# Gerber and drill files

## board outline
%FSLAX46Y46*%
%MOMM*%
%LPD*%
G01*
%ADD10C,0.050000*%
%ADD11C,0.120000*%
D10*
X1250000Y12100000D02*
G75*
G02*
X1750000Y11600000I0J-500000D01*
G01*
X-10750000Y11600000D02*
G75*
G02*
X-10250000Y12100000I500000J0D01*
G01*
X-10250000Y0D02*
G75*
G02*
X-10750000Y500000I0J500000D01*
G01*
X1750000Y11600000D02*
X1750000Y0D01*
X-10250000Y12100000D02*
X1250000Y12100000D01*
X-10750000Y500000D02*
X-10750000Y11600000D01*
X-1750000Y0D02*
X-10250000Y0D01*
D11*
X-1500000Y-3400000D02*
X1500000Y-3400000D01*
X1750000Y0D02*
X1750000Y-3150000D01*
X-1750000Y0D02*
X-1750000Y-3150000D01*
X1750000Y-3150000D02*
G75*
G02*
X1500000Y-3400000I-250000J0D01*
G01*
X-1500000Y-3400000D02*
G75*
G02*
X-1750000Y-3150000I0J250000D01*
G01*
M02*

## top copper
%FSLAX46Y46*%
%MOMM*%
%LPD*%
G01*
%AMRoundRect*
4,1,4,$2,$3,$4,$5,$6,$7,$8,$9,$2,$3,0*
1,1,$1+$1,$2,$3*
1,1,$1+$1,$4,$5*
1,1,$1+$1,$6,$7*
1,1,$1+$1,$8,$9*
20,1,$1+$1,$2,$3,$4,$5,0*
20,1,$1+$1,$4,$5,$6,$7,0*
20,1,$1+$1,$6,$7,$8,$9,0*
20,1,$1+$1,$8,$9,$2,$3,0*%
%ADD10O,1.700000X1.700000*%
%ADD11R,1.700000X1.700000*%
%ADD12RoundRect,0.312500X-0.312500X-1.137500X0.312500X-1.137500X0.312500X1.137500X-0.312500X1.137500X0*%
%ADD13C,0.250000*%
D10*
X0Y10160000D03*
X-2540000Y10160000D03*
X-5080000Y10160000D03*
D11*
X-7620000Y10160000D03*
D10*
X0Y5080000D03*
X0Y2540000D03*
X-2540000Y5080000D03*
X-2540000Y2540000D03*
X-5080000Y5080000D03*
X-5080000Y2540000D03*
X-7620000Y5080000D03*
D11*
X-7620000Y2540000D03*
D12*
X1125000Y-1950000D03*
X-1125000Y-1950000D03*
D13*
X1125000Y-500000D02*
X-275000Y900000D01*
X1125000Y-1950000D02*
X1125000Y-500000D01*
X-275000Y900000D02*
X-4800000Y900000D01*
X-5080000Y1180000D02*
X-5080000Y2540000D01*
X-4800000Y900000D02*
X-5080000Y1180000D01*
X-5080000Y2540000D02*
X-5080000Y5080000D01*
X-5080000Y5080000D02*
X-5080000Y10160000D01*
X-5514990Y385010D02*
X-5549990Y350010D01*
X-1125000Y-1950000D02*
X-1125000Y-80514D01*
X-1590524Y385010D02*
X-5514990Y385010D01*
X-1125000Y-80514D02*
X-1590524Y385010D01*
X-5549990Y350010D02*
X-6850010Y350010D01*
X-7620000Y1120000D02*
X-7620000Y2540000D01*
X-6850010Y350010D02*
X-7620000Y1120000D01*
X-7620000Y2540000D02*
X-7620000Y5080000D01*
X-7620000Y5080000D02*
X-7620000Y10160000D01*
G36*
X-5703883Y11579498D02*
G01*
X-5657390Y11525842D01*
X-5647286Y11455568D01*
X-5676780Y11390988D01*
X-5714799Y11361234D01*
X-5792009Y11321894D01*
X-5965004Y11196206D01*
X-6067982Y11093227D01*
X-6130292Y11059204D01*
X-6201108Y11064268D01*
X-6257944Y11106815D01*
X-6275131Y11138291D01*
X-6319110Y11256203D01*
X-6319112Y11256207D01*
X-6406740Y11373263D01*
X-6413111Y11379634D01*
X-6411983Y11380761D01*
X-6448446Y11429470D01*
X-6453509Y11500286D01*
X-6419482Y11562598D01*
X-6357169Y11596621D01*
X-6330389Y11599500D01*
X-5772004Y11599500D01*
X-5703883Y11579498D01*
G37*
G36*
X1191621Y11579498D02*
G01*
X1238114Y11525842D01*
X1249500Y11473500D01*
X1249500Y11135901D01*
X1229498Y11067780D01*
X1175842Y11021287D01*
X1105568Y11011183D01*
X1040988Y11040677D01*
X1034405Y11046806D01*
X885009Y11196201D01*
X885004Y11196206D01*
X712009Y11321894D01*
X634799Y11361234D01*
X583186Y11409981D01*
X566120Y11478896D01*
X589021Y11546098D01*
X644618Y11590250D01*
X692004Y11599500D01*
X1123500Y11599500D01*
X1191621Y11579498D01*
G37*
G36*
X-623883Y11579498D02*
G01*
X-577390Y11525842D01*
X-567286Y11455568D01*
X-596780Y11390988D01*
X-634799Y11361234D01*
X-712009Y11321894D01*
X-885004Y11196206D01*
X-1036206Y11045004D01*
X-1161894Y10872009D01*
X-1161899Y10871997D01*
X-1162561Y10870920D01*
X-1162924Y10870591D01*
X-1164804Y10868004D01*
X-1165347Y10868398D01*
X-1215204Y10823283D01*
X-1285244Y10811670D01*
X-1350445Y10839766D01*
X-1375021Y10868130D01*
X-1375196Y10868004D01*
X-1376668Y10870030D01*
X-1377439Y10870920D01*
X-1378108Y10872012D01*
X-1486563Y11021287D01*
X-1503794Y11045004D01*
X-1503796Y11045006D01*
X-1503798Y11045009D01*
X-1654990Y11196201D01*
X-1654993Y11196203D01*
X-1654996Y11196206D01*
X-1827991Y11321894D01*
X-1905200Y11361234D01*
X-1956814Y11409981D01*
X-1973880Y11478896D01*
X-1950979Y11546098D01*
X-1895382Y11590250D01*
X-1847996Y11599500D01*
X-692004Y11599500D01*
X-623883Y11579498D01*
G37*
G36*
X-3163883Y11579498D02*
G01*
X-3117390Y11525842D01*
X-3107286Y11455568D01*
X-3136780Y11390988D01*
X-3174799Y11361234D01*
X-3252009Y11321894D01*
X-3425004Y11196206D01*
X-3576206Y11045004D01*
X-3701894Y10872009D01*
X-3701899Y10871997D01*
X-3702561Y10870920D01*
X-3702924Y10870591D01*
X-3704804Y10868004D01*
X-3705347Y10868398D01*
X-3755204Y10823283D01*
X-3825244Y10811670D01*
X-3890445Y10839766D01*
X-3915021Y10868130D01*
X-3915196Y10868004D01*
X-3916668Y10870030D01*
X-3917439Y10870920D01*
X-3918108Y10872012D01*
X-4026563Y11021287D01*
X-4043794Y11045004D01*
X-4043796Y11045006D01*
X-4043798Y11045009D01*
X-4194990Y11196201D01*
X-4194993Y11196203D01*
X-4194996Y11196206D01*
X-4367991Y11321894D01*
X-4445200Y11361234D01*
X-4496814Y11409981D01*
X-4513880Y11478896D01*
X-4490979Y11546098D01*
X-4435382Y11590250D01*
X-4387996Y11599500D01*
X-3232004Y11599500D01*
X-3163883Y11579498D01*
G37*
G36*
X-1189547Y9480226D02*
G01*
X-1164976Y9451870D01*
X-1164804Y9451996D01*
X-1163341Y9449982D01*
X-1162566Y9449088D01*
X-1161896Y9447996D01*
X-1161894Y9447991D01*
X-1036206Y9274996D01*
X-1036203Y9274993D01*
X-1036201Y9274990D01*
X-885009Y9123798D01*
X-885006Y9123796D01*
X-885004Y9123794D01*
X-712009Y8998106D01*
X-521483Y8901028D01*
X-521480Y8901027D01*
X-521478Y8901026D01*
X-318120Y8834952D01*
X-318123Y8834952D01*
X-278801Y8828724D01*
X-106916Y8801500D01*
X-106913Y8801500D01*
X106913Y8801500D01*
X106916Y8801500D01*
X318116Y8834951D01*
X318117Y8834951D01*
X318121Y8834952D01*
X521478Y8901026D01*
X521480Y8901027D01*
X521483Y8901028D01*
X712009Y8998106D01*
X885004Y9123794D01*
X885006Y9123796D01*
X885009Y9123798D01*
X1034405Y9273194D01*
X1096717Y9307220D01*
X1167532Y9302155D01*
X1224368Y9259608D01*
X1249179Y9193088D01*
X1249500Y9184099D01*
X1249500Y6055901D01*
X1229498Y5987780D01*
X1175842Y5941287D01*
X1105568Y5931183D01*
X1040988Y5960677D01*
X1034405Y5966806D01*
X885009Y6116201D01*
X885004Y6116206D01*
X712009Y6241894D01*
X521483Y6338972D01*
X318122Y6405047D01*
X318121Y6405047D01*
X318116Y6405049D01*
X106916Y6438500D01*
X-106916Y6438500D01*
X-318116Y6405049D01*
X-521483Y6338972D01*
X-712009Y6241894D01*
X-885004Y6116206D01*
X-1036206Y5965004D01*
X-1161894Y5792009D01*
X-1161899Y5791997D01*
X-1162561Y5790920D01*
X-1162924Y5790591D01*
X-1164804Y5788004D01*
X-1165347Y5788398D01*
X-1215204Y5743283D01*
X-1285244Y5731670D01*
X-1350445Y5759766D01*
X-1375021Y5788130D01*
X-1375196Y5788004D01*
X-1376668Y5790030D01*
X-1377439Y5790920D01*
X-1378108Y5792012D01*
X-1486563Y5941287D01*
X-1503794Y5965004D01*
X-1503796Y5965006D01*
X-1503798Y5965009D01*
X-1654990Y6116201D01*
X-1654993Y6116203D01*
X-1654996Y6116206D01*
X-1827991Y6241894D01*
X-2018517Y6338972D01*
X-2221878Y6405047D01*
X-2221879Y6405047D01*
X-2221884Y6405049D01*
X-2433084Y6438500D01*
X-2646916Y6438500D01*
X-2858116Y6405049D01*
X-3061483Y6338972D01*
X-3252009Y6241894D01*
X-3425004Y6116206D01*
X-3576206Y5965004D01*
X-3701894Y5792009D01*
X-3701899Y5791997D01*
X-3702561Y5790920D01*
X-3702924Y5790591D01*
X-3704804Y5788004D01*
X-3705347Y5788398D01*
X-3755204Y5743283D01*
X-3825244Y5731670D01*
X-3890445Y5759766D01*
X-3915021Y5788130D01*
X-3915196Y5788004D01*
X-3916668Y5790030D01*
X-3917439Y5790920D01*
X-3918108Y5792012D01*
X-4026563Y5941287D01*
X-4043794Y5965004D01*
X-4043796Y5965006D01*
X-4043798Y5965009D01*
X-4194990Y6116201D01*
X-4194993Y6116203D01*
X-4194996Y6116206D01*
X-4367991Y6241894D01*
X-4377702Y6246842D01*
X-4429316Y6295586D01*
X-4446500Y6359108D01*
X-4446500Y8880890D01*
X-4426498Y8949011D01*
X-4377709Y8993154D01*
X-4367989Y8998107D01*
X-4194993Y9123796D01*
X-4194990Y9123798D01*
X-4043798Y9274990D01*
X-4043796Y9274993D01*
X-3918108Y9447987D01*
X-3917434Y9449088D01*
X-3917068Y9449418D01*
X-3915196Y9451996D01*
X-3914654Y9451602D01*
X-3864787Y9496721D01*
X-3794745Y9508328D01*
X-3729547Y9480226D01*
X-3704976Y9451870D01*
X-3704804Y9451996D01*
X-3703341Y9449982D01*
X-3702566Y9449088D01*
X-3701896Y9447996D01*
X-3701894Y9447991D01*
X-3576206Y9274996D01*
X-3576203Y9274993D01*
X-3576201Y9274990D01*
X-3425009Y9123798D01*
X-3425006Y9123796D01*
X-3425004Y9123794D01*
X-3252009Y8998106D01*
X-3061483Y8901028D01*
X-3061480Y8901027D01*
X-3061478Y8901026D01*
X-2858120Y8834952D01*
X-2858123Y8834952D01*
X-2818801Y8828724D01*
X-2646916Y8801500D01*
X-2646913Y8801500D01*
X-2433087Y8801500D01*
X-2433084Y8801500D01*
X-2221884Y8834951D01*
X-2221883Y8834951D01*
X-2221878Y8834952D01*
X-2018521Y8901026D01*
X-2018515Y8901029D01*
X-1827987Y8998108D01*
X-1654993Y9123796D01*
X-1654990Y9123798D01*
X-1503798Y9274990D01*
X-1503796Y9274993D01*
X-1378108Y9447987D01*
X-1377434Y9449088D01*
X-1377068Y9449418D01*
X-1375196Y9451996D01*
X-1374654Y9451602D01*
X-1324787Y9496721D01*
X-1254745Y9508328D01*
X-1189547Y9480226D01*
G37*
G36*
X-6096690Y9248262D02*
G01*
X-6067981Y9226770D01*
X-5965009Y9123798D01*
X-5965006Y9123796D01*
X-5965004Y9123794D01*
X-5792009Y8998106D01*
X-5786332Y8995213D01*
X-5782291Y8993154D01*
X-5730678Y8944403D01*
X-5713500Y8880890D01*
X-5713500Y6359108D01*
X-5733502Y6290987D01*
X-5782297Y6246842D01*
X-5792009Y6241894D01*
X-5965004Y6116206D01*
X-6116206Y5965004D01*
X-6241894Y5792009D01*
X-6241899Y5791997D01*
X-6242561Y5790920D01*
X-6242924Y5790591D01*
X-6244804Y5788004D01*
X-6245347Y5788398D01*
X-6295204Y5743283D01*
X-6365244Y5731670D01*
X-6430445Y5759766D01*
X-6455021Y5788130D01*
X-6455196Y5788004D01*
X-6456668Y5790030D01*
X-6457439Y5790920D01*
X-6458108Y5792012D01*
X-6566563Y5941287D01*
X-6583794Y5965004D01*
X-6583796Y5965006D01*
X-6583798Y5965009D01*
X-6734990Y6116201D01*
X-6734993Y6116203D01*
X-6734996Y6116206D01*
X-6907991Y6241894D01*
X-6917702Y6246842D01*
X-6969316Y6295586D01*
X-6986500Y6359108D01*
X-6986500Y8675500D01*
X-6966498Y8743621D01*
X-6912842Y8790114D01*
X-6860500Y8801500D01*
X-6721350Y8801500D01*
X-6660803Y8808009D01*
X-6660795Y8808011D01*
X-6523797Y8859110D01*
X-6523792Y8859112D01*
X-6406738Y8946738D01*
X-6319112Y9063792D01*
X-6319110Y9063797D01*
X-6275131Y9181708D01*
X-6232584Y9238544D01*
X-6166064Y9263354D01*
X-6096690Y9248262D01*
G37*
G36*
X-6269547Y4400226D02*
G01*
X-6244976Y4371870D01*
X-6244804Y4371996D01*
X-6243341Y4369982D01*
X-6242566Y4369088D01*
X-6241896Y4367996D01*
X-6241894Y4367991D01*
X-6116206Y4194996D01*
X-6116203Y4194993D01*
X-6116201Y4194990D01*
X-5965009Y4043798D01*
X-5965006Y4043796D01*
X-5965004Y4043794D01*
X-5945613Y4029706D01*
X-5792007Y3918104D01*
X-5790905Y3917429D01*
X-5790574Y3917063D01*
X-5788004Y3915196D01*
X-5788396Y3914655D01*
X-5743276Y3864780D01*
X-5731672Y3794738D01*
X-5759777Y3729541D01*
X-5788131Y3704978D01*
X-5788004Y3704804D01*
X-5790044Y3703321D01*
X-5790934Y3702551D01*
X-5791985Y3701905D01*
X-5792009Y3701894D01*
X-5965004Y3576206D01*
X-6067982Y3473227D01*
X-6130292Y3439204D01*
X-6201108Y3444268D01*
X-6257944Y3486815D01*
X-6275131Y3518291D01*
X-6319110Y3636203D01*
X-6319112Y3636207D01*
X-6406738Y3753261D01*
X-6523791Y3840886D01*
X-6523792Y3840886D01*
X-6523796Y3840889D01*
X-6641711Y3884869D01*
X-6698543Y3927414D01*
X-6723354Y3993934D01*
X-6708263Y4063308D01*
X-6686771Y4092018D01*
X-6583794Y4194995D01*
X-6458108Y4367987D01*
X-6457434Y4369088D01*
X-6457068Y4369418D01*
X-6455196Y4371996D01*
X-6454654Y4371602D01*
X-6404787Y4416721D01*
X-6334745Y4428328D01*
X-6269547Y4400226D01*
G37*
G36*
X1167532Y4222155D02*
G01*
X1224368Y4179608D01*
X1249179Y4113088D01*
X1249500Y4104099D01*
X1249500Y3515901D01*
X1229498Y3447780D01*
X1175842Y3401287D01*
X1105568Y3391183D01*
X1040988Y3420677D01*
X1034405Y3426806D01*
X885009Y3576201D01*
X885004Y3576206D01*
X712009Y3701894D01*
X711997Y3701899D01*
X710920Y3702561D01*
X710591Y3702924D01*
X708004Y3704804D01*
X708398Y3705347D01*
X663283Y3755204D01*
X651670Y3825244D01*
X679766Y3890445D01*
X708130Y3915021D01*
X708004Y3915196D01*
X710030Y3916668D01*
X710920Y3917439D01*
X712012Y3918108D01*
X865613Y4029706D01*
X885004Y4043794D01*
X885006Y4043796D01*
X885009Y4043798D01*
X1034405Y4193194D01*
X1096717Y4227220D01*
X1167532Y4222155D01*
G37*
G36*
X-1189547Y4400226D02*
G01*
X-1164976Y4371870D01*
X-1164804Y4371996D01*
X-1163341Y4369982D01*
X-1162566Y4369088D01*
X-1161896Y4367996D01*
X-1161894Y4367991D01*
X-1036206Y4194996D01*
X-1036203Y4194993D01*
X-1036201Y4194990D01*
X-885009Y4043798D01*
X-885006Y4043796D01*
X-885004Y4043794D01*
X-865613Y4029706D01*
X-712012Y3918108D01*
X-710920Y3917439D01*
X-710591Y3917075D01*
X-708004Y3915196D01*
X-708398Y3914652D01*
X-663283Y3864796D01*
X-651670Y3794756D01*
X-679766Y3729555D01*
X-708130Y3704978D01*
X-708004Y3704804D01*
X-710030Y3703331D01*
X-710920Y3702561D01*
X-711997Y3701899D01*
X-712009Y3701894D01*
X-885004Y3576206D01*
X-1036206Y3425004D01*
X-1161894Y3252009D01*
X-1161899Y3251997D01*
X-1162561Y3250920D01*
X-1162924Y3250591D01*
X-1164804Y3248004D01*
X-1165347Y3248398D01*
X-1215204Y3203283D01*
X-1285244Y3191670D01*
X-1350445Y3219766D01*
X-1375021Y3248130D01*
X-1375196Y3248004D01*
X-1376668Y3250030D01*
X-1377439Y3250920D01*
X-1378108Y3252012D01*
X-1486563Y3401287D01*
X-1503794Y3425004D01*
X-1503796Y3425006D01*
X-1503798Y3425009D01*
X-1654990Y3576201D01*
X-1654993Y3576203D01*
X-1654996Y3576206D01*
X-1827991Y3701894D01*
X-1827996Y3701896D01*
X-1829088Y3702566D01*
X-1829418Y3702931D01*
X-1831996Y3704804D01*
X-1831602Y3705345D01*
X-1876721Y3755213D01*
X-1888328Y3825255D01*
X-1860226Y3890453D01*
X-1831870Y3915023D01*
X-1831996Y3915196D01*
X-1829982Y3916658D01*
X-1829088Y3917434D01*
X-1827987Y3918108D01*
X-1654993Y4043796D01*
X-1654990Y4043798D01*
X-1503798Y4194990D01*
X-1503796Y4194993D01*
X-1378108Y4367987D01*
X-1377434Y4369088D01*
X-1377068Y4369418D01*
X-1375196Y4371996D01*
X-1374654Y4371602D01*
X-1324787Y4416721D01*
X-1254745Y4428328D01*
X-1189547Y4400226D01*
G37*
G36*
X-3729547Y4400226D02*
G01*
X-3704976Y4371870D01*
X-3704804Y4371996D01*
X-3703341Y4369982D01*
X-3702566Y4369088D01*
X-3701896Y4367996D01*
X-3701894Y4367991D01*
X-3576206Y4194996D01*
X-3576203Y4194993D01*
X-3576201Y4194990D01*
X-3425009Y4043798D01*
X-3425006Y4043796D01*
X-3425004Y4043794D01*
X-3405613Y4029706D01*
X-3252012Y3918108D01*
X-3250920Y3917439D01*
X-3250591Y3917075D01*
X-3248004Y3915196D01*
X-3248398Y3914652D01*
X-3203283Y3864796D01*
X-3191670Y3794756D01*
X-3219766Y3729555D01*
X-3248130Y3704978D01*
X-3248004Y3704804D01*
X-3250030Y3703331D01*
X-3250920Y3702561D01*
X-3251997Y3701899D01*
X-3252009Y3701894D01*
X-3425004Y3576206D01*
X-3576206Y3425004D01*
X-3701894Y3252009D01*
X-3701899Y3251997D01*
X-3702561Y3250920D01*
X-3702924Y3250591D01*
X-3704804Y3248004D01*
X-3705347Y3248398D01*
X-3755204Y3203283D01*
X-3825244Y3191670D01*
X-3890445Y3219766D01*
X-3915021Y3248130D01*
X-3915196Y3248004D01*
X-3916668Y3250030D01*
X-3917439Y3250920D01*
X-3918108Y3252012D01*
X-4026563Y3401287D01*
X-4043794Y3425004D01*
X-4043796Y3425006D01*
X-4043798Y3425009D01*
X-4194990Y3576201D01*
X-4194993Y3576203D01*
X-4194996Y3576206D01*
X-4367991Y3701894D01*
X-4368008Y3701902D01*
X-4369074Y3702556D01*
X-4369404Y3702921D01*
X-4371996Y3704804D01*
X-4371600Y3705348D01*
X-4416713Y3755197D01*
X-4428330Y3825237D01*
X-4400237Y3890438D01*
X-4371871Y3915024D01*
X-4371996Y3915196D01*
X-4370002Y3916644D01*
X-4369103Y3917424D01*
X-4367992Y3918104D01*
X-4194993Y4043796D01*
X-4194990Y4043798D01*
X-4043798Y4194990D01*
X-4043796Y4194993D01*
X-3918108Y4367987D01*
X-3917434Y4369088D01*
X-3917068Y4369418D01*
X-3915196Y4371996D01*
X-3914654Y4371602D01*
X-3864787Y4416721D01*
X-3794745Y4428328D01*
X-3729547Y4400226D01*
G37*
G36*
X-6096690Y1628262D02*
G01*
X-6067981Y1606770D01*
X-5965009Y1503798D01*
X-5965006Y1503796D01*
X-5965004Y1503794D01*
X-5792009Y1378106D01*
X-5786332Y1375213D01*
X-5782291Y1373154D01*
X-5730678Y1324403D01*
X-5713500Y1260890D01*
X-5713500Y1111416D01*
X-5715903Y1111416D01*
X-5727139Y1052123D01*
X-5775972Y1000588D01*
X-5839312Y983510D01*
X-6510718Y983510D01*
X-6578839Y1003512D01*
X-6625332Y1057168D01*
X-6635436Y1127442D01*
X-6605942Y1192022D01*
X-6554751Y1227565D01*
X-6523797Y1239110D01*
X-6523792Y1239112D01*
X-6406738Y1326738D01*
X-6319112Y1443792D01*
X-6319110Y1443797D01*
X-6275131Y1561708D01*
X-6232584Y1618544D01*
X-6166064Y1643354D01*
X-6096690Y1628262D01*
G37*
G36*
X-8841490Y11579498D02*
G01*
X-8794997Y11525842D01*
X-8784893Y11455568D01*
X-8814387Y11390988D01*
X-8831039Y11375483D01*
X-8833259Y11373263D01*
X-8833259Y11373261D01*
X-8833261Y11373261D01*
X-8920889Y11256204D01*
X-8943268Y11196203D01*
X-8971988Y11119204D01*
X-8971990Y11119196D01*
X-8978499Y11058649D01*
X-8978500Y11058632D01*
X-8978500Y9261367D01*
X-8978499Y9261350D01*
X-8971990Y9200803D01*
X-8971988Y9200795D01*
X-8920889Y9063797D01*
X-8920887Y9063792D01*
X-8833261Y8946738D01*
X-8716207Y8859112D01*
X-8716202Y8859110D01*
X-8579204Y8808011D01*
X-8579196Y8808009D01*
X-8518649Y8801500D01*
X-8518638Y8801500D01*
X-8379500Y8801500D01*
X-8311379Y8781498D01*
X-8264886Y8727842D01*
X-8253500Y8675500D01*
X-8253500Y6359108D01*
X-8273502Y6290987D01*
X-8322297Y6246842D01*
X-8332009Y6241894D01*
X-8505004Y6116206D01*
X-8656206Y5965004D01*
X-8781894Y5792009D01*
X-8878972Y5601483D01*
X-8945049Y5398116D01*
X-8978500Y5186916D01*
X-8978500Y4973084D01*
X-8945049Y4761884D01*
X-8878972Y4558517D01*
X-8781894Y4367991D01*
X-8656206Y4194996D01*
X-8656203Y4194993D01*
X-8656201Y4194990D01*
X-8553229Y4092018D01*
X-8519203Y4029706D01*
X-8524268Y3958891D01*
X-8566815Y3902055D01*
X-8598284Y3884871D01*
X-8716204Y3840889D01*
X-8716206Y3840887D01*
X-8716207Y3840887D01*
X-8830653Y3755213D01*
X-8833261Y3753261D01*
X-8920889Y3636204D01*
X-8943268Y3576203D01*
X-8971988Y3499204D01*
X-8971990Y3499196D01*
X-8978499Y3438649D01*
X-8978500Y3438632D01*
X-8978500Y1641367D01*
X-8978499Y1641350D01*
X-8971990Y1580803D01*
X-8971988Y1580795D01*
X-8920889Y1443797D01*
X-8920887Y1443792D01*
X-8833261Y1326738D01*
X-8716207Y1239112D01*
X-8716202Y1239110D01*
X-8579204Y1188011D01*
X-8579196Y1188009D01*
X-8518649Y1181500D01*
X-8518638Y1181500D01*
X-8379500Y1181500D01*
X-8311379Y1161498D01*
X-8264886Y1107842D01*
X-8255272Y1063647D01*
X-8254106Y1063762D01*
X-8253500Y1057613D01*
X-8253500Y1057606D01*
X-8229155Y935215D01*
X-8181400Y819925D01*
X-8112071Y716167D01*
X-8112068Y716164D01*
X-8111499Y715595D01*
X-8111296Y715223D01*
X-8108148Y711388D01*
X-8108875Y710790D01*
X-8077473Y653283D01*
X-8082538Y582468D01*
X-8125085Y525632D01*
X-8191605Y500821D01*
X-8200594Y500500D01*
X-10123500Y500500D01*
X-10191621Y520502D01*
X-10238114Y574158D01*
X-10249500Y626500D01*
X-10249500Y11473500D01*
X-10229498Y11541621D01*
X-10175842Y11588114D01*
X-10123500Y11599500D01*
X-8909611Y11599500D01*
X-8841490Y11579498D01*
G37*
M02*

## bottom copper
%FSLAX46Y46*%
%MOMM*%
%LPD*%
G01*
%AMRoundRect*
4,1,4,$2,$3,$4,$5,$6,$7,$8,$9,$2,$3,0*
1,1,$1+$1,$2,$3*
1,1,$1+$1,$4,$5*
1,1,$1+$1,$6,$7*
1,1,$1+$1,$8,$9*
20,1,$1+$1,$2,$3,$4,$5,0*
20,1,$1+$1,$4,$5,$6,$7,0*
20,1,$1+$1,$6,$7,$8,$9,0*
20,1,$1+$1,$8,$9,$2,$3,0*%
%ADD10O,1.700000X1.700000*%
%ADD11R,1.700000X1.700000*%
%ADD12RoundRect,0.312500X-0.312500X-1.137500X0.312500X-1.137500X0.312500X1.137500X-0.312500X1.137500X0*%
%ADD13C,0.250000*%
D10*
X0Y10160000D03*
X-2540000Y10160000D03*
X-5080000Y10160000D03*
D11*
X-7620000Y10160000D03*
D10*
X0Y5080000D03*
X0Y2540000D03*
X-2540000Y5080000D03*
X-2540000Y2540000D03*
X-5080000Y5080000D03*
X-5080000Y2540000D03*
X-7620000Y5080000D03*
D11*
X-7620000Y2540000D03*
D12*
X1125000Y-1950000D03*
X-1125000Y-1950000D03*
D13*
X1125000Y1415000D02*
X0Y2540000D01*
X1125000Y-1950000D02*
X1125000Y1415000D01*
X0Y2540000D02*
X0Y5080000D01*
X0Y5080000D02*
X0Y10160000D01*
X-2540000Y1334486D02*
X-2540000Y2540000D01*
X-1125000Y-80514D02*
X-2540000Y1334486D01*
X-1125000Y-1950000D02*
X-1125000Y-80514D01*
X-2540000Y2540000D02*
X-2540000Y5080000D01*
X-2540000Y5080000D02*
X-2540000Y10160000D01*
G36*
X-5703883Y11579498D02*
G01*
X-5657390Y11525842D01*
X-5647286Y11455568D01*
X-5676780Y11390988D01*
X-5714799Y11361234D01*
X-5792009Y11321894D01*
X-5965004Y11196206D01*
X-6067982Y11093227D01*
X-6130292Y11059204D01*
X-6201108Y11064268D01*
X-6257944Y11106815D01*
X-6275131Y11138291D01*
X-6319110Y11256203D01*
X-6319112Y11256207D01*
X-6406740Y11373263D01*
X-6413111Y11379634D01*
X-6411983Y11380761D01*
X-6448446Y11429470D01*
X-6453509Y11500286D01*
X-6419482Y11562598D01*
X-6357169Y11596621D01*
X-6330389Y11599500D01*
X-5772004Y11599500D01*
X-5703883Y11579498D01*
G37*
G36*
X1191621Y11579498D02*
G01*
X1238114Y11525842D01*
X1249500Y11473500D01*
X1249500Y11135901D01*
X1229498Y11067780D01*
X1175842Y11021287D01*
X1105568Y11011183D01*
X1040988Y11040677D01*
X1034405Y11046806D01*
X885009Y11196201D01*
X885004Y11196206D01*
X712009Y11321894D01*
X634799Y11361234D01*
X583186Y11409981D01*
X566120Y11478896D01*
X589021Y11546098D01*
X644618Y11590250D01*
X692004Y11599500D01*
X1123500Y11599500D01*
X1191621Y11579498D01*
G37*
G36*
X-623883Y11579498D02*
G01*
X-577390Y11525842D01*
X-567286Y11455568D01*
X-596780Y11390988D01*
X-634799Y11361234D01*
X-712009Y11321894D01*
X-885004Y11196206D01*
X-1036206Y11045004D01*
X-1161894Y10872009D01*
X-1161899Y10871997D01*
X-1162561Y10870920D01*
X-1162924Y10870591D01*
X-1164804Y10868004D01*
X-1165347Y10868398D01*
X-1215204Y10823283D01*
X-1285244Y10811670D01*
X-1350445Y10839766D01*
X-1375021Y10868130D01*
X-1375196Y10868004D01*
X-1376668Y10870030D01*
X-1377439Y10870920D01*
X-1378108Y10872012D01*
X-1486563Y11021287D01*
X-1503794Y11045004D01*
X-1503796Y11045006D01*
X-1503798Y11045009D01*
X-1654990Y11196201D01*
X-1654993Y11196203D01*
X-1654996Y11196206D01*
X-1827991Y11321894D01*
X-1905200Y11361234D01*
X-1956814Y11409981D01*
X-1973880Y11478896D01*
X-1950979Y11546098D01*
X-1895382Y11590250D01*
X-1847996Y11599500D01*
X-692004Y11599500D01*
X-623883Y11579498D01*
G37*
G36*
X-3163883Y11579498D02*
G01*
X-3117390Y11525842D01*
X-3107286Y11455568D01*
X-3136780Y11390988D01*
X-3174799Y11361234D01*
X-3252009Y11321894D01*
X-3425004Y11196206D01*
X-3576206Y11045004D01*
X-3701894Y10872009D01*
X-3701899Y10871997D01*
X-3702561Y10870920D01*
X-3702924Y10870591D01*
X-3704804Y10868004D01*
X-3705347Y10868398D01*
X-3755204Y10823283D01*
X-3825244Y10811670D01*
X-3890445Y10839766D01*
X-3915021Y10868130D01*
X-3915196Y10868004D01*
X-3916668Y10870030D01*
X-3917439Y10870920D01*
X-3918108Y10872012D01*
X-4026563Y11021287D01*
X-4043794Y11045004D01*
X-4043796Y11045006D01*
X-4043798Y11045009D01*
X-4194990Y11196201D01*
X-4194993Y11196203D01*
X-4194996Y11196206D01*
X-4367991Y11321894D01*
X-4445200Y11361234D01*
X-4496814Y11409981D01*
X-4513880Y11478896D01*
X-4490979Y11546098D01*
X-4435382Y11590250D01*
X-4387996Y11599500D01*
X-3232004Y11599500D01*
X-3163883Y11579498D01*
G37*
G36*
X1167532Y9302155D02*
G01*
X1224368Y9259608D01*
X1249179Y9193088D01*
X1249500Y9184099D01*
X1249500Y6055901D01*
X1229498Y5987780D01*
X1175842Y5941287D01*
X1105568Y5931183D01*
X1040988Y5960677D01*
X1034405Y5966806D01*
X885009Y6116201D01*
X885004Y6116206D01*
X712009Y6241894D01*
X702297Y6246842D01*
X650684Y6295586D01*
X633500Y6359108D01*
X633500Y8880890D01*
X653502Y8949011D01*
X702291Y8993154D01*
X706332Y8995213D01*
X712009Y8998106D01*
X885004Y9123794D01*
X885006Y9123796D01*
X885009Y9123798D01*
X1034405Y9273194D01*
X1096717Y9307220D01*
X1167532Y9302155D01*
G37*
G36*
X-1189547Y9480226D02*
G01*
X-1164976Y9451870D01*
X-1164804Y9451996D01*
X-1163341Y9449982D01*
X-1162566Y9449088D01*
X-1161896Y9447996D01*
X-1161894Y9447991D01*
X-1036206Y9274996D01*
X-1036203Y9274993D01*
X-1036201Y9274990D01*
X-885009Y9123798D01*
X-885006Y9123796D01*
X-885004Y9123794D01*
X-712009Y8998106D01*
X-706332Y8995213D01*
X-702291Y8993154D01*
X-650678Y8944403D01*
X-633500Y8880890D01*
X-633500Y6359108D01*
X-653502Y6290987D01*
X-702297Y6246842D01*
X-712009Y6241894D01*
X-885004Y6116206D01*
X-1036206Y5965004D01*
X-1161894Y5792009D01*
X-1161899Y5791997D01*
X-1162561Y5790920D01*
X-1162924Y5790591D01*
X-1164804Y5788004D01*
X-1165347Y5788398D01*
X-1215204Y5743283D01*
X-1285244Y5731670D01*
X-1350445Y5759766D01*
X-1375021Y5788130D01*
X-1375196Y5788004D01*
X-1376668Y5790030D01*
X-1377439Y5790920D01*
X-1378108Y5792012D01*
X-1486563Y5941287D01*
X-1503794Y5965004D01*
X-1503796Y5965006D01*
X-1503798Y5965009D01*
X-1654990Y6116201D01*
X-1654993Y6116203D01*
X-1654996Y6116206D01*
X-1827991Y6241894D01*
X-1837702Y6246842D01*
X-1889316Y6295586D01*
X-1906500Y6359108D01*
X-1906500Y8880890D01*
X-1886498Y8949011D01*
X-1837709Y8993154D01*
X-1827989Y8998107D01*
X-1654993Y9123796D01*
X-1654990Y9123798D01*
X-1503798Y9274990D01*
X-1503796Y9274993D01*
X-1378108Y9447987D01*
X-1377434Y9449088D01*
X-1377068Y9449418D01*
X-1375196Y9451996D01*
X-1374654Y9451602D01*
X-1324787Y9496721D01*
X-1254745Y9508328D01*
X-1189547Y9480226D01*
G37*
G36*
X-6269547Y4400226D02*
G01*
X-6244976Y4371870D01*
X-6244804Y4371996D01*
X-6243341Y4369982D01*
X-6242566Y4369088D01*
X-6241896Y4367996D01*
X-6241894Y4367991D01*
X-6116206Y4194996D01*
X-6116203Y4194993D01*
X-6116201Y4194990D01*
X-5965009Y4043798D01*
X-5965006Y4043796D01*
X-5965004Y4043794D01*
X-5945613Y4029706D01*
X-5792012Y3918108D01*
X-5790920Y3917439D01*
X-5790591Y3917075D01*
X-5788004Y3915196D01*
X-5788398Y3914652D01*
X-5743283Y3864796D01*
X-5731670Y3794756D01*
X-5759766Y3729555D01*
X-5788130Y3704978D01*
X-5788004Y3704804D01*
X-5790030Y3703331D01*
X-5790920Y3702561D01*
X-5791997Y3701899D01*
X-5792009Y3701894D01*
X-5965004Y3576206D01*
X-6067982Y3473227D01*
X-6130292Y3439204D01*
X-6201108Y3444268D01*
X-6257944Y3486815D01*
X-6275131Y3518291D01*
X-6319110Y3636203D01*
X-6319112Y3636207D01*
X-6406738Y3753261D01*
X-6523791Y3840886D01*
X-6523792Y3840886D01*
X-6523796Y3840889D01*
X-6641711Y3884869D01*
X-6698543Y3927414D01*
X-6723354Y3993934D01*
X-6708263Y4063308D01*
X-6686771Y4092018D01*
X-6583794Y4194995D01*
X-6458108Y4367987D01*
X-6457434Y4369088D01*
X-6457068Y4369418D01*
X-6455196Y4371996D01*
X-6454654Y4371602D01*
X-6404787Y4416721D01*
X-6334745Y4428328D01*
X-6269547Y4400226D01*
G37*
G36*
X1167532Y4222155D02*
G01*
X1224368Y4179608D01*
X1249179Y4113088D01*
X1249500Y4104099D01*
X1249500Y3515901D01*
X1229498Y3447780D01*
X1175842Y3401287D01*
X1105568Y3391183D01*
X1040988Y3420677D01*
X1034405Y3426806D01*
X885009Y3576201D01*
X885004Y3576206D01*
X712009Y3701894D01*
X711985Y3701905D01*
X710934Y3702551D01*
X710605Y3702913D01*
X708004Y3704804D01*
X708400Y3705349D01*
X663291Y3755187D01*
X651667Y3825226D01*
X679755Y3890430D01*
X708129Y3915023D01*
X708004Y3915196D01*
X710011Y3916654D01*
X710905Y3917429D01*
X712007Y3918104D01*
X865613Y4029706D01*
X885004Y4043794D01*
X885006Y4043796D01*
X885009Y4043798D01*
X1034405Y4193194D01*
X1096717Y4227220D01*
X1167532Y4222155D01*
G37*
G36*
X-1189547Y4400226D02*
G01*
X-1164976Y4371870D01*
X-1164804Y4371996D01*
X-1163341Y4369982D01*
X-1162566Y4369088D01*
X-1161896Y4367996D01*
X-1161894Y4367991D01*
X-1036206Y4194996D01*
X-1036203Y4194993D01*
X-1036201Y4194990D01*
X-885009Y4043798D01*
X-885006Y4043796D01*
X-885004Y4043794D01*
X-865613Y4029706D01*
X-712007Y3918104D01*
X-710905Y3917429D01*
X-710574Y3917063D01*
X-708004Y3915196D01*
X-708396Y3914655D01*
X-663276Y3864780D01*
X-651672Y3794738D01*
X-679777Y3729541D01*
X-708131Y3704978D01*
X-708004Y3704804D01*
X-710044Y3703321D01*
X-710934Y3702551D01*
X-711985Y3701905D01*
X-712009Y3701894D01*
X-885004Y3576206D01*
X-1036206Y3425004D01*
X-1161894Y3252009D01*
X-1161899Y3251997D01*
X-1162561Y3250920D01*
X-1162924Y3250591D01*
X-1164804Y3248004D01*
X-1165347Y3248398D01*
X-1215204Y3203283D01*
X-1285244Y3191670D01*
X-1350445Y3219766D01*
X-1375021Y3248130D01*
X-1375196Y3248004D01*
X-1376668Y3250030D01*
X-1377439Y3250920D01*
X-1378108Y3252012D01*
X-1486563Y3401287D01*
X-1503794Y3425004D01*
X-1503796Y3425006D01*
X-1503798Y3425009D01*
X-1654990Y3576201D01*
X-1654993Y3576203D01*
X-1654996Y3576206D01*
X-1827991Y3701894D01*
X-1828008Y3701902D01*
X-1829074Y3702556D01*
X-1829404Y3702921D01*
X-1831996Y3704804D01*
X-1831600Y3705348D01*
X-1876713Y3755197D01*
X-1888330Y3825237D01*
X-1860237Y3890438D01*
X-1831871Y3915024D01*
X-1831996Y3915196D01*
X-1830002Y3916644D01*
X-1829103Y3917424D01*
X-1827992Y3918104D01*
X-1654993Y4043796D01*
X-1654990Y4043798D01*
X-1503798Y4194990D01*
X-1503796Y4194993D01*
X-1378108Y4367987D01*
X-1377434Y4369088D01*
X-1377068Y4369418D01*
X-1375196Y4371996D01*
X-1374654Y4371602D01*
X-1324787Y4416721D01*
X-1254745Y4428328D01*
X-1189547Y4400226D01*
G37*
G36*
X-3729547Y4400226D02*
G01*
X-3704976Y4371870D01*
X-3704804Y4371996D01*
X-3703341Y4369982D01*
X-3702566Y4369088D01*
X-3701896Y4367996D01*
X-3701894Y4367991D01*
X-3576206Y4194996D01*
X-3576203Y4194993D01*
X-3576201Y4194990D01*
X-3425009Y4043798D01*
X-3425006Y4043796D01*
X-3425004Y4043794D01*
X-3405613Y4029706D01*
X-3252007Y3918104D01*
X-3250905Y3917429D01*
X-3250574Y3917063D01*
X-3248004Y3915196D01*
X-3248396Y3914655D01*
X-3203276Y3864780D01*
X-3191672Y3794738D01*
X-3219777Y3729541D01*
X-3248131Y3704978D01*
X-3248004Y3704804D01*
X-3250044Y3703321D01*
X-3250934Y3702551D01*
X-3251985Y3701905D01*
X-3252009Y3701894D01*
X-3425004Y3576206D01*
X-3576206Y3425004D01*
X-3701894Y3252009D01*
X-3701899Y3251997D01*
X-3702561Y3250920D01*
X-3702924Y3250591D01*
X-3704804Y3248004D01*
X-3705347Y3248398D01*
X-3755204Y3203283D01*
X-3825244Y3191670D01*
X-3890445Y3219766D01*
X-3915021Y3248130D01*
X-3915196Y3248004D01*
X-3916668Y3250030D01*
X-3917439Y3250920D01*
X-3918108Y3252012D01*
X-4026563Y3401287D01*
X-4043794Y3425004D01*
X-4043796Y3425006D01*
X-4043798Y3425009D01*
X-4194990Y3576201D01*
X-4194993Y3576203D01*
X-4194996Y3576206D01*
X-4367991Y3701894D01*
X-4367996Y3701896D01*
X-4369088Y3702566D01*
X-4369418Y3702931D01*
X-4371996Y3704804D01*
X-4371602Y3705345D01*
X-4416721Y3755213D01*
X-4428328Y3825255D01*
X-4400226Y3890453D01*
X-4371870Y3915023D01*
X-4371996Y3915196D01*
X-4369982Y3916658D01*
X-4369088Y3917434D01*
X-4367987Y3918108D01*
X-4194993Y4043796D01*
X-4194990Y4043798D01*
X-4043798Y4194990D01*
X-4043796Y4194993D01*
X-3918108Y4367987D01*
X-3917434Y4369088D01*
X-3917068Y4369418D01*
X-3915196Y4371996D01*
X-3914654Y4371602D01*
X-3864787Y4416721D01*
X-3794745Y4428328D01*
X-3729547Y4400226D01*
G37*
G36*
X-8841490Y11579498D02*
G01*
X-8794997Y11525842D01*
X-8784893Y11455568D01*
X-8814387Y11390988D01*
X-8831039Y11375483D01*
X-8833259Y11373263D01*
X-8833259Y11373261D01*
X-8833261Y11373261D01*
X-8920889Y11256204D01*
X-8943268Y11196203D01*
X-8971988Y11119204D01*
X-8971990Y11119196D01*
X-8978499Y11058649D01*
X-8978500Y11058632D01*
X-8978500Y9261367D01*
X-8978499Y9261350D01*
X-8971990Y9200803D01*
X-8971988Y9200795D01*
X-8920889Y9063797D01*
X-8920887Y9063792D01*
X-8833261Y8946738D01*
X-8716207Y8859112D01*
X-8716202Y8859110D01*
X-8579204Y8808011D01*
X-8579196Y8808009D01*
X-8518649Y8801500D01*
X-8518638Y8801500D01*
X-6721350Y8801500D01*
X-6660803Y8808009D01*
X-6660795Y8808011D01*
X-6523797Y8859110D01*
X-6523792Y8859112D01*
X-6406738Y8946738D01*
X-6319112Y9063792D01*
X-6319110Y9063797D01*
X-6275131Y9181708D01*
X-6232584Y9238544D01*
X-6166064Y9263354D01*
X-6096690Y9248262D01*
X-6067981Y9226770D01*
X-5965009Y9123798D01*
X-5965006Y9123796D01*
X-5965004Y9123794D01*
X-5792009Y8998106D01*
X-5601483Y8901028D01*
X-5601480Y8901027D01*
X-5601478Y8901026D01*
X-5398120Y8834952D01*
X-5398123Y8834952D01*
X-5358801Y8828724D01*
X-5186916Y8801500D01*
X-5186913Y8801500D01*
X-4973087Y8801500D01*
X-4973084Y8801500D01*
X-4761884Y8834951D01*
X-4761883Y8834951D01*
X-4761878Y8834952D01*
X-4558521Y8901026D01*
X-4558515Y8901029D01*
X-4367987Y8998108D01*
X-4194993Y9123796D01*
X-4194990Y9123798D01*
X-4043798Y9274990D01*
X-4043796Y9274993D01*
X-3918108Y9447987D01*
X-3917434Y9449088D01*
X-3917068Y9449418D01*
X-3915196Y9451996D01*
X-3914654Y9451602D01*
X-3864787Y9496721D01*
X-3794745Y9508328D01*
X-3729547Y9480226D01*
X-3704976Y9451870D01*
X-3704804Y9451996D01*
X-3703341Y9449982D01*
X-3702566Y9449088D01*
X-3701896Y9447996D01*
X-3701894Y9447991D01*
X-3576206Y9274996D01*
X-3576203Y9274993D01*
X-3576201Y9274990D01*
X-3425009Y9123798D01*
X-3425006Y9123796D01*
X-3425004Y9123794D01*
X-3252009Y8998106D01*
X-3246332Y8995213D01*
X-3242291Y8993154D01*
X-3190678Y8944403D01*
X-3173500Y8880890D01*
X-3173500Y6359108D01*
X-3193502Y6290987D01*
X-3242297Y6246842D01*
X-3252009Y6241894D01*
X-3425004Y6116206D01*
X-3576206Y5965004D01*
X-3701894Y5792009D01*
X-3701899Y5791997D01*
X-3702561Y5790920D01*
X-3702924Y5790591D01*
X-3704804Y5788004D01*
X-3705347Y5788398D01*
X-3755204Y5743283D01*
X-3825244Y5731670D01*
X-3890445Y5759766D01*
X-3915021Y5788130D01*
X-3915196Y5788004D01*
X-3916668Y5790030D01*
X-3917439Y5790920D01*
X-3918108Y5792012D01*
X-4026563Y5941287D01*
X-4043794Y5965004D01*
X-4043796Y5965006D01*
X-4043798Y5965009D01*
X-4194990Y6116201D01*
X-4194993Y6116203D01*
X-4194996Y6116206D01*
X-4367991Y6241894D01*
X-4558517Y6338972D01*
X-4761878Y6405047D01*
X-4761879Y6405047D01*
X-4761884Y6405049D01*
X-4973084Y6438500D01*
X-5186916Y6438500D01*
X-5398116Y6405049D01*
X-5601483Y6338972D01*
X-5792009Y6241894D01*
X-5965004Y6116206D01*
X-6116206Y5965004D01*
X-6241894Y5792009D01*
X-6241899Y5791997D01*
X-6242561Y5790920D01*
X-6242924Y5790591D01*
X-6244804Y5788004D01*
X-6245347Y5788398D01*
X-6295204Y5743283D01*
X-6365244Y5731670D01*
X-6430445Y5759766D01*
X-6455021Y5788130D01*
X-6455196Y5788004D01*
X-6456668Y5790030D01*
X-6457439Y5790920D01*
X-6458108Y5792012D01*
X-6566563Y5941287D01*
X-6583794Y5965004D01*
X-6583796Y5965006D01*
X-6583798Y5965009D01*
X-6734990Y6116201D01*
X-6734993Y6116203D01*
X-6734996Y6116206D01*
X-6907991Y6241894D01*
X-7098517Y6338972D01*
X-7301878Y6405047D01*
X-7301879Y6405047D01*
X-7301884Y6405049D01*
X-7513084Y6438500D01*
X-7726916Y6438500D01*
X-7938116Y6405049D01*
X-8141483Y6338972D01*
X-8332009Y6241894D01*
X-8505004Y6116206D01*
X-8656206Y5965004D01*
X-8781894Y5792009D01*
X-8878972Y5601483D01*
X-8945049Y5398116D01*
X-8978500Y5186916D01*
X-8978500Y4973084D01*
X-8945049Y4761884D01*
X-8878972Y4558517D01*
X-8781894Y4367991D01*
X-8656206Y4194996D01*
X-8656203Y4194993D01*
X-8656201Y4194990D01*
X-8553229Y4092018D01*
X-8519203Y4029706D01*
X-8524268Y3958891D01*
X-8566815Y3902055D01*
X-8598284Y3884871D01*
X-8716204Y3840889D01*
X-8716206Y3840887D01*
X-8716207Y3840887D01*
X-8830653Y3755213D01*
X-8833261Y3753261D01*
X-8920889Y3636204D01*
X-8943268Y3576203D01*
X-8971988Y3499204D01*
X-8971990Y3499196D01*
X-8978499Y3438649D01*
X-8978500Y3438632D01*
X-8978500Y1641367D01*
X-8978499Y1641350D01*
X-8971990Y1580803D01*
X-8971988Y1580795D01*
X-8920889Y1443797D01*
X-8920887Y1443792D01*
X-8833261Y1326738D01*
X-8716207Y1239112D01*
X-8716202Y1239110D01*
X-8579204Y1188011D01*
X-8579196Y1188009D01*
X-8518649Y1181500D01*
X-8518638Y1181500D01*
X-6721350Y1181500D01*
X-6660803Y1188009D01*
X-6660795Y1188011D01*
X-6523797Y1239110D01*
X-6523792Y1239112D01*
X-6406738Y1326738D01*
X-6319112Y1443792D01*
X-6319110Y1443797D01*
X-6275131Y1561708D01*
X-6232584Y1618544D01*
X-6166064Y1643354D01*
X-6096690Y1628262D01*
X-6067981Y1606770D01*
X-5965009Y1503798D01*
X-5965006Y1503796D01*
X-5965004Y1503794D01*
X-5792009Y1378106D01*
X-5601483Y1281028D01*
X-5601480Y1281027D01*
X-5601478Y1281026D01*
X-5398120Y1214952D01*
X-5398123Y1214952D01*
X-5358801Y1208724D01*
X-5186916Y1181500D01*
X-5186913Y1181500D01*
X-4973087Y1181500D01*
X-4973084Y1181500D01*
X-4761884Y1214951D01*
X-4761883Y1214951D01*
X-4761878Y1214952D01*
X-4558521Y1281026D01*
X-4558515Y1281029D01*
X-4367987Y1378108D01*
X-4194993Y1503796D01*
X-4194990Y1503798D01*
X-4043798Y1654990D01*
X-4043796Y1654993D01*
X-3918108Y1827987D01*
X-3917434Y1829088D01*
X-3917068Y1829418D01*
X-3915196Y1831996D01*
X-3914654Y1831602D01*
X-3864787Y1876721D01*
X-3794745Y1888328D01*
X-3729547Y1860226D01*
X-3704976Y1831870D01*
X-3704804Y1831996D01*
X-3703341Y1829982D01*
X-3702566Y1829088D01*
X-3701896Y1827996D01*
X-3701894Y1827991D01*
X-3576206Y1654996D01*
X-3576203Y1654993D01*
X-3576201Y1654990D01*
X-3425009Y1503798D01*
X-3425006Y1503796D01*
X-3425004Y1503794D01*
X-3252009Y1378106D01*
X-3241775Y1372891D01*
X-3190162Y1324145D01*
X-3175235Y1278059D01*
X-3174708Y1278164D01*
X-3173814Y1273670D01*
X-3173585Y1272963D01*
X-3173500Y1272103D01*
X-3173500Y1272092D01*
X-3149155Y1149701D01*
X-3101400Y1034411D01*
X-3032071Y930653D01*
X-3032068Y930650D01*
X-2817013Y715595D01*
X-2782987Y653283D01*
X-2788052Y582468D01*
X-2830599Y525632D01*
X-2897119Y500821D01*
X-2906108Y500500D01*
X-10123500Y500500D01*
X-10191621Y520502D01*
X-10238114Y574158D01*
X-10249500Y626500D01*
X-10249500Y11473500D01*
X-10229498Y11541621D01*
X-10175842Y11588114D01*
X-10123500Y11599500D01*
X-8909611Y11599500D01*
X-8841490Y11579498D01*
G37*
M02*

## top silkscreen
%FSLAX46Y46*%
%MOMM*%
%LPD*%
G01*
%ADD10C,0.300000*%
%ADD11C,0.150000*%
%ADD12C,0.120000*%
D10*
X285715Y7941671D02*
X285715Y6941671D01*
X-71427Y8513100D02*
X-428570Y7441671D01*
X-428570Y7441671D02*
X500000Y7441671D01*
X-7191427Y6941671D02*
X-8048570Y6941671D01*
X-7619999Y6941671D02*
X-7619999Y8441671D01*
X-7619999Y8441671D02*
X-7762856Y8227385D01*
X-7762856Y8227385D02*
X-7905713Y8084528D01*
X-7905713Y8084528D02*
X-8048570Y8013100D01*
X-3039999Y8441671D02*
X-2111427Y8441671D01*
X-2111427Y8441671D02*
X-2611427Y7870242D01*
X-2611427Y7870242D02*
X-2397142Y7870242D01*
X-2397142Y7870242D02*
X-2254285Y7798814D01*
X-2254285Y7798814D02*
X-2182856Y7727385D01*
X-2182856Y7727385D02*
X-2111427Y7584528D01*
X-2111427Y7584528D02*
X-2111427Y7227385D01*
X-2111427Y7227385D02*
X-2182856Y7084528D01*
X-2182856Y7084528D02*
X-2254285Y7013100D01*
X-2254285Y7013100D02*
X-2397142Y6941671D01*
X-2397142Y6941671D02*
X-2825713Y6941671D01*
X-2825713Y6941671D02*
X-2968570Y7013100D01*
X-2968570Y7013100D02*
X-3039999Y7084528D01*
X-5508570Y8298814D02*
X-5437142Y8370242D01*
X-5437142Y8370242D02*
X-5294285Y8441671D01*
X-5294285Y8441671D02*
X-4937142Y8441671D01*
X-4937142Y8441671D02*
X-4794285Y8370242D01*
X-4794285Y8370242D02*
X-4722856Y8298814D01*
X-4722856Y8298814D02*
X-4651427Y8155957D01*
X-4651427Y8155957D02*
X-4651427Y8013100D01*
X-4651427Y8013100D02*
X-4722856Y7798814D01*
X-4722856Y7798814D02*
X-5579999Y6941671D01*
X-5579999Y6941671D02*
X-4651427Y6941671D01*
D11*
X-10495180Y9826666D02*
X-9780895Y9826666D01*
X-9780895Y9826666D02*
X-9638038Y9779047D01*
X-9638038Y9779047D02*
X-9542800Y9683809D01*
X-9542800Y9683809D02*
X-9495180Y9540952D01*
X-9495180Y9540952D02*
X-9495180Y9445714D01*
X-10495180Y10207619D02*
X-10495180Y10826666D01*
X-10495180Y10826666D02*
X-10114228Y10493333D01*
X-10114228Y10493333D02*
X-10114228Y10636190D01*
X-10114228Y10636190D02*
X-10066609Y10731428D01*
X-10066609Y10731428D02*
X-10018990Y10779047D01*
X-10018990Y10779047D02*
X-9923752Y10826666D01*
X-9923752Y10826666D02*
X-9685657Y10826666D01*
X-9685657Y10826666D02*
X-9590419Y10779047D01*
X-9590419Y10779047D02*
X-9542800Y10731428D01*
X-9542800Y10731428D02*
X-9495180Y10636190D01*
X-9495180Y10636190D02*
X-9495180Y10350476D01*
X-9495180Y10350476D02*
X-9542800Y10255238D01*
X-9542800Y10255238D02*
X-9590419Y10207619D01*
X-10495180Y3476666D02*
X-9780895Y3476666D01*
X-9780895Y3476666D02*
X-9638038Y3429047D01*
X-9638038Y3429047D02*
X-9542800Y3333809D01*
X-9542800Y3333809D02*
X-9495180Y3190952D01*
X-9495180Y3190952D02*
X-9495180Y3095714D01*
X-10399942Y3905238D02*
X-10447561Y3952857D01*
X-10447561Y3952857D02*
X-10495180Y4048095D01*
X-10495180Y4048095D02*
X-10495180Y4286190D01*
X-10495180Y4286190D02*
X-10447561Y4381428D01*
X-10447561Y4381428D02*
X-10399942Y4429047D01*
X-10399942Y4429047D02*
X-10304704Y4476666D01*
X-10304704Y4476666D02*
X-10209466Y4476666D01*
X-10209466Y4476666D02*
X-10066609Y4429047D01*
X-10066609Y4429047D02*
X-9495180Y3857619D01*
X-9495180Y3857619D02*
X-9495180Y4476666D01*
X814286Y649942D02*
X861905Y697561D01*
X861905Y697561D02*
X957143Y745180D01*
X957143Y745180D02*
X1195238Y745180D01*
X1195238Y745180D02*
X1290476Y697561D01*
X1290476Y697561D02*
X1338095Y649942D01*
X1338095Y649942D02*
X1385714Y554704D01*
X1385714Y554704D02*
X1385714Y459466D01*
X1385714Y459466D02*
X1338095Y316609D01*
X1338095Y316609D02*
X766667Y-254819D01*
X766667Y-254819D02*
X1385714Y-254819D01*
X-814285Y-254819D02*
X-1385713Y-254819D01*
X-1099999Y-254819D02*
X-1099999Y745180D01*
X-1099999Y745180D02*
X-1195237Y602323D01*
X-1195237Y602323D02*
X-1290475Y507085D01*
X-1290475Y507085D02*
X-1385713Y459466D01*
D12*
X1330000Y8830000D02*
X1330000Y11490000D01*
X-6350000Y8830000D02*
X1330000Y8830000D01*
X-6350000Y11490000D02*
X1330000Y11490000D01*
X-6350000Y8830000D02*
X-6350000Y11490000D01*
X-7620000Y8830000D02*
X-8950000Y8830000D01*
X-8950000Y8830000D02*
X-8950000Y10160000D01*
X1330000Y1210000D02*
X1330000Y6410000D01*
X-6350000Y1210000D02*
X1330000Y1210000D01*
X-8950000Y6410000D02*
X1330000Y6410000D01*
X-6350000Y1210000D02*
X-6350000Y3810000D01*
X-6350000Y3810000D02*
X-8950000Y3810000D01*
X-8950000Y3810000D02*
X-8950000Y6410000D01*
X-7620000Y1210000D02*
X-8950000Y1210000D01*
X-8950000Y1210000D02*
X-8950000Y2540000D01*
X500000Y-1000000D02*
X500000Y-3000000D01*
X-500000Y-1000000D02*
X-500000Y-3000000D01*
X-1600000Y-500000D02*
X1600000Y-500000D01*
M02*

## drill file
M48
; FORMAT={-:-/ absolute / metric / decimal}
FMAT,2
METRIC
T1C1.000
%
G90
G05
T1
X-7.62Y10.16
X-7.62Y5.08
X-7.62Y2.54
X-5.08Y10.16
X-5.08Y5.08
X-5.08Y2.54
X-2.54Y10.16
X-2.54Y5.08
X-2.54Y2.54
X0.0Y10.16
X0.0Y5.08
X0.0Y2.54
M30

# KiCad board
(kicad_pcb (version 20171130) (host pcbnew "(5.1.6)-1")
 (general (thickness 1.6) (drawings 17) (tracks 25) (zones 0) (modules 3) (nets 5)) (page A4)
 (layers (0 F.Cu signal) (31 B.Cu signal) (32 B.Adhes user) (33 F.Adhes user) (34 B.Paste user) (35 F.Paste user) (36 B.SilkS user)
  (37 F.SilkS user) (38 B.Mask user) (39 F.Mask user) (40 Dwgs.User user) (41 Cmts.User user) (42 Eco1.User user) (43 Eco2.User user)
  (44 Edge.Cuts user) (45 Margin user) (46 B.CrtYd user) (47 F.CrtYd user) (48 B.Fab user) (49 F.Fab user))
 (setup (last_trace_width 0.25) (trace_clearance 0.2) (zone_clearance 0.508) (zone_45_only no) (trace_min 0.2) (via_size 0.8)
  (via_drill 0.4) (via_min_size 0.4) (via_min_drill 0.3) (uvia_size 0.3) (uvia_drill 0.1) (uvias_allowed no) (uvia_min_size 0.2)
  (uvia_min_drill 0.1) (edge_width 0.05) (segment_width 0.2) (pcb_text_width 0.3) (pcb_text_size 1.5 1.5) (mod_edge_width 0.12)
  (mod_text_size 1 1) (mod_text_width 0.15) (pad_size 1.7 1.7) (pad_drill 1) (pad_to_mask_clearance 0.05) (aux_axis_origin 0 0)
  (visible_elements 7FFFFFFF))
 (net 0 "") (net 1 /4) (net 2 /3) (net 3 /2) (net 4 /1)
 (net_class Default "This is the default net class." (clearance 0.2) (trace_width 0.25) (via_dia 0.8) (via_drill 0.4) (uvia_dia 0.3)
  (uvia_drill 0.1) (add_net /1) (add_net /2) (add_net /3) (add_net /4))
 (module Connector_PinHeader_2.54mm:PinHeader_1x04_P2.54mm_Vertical (layer F.Cu) (at -7.62 -10.16 90)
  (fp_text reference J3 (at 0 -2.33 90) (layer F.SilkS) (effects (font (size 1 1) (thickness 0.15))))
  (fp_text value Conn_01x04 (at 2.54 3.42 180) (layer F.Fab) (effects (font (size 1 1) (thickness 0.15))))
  (fp_line (start -1.33 8.95) (end 1.33 8.95) (layer F.SilkS) (width 0.12))
  (fp_line (start -1.33 1.27) (end -1.33 8.95) (layer F.SilkS) (width 0.12))
  (fp_line (start 1.33 1.27) (end 1.33 8.95) (layer F.SilkS) (width 0.12))
  (fp_line (start -1.33 1.27) (end 1.33 1.27) (layer F.SilkS) (width 0.12))
  (fp_line (start -1.33 0) (end -1.33 -1.33) (layer F.SilkS) (width 0.12))
  (fp_line (start -1.33 -1.33) (end 0 -1.33) (layer F.SilkS) (width 0.12))
  (pad 4 thru_hole oval (at 0 7.62 90) (size 1.7 1.7) (drill 1) (layers *.Cu *.Mask) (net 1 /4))
  (pad 3 thru_hole oval (at 0 5.08 90) (size 1.7 1.7) (drill 1) (layers *.Cu *.Mask) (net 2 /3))
  (pad 2 thru_hole oval (at 0 2.54 90) (size 1.7 1.7) (drill 1) (layers *.Cu *.Mask) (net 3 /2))
  (pad 1 thru_hole rect (at 0 0 90) (size 1.7 1.7) (drill 1) (layers *.Cu *.Mask) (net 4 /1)))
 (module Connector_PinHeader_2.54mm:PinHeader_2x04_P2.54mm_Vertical (layer F.Cu) (at -7.62 -2.54 90)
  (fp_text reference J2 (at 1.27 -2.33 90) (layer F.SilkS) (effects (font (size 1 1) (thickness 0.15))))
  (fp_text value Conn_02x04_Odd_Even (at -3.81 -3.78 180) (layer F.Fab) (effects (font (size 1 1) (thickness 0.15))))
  (fp_line (start -1.33 8.95) (end 3.87 8.95) (layer F.SilkS) (width 0.12))
  (fp_line (start -1.33 1.27) (end -1.33 8.95) (layer F.SilkS) (width 0.12))
  (fp_line (start 3.87 -1.33) (end 3.87 8.95) (layer F.SilkS) (width 0.12))
  (fp_line (start -1.33 1.27) (end 1.27 1.27) (layer F.SilkS) (width 0.12))
  (fp_line (start 1.27 1.27) (end 1.27 -1.33) (layer F.SilkS) (width 0.12))
  (fp_line (start 1.27 -1.33) (end 3.87 -1.33) (layer F.SilkS) (width 0.12))
  (fp_line (start -1.33 0) (end -1.33 -1.33) (layer F.SilkS) (width 0.12))
  (fp_line (start -1.33 -1.33) (end 0 -1.33) (layer F.SilkS) (width 0.12))
  (pad 8 thru_hole oval (at 2.54 7.62 90) (size 1.7 1.7) (drill 1) (layers *.Cu *.Mask) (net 1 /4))
  (pad 7 thru_hole oval (at 0 7.62 90) (size 1.7 1.7) (drill 1) (layers *.Cu *.Mask) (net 1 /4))
  (pad 6 thru_hole oval (at 2.54 5.08 90) (size 1.7 1.7) (drill 1) (layers *.Cu *.Mask) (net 2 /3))
  (pad 5 thru_hole oval (at 0 5.08 90) (size 1.7 1.7) (drill 1) (layers *.Cu *.Mask) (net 2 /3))
  (pad 4 thru_hole oval (at 2.54 2.54 90) (size 1.7 1.7) (drill 1) (layers *.Cu *.Mask) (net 3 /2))
  (pad 3 thru_hole oval (at 0 2.54 90) (size 1.7 1.7) (drill 1) (layers *.Cu *.Mask) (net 3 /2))
  (pad 2 thru_hole oval (at 2.54 0 90) (size 1.7 1.7) (drill 1) (layers *.Cu *.Mask) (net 4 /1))
  (pad 1 thru_hole rect (at 0 0 90) (size 1.7 1.7) (drill 1) (layers *.Cu *.Mask) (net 4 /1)))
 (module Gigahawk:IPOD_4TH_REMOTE (layer F.Cu) (at 0 0)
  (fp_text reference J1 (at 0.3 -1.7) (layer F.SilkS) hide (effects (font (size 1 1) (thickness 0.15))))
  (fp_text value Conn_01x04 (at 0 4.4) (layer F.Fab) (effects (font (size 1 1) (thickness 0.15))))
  (fp_line (start 0.5 1) (end 0.5 3) (layer F.SilkS) (width 0.12))
  (fp_line (start -0.5 1) (end -0.5 3) (layer F.SilkS) (width 0.12))
  (fp_line (start -1.6 0.5) (end 1.6 0.5) (layer F.SilkS) (width 0.12))
  (fp_line (start -1.5 3.4) (end 1.5 3.4) (layer Edge.Cuts) (width 0.12))
  (fp_line (start 1.75 0) (end 1.75 3.15) (layer Edge.Cuts) (width 0.12))
  (fp_line (start -1.75 0) (end -1.75 3.15) (layer Edge.Cuts) (width 0.12))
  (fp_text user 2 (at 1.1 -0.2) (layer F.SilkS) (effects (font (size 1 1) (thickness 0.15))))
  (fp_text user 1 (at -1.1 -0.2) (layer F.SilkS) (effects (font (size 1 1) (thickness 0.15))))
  (fp_arc (start 1.5 3.15) (end 1.75 3.15) (angle 90) (layer Edge.Cuts) (width 0.12))
  (fp_arc (start -1.5 3.15) (end -1.75 3.15) (angle -90) (layer Edge.Cuts) (width 0.12))
  (pad 2 connect roundrect (at 1.125 1.95) (size 1.25 2.9) (layers F.Cu F.Mask) (roundrect_rratio 0.25) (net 3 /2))
  (pad 1 connect roundrect (at -1.125 1.95) (size 1.25 2.9) (layers F.Cu F.Mask) (roundrect_rratio 0.25) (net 4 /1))
  (pad 4 connect roundrect (at 1.125 1.95) (size 1.25 2.9) (layers B.Cu B.Mask) (roundrect_rratio 0.25) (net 1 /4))
  (pad 3 connect roundrect (at -1.125 1.95) (size 1.25 2.9) (layers B.Cu B.Mask) (roundrect_rratio 0.25) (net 2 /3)))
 (gr_arc (start 1.25 -11.6) (end 1.75 -11.6) (angle -90) (layer Edge.Cuts) (width 0.05))
 (gr_arc (start -10.25 -11.6) (end -10.75 -11.6) (angle 90) (layer Edge.Cuts) (width 0.05))
 (gr_arc (start -10.25 -0.5) (end -10.75 -0.5) (angle -90) (layer Edge.Cuts) (width 0.05))
 (gr_line (start 1.75 -11.6) (end 1.75 0) (layer Edge.Cuts) (width 0.05))
 (gr_line (start -10.25 -12.1) (end 1.25 -12.1) (layer Edge.Cuts) (width 0.05))
 (gr_line (start -10.75 -0.5) (end -10.75 -11.6) (layer Edge.Cuts) (width 0.05))
 (gr_line (start -1.75 0) (end -10.25 0) (layer Edge.Cuts) (width 0.05))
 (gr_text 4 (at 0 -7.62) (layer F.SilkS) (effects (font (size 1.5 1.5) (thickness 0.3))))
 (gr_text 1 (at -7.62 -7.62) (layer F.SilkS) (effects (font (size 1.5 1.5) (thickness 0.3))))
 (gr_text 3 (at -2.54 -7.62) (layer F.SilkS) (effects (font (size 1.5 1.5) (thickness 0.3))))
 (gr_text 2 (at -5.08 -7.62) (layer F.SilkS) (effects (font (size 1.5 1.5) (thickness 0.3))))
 (segment (start 1.125 0.5) (end -0.275 -0.9) (width 0.25) (layer F.Cu) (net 3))
 (segment (start 1.125 1.95) (end 1.125 0.5) (width 0.25) (layer F.Cu) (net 3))
 (segment (start -0.275 -0.9) (end -4.8 -0.9) (width 0.25) (layer F.Cu) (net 3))
 (segment (start -5.08 -1.18) (end -5.08 -2.54) (width 0.25) (layer F.Cu) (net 3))
 (segment (start -4.8 -0.9) (end -5.08 -1.18) (width 0.25) (layer F.Cu) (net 3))
 (segment (start -5.08 -2.54) (end -5.08 -5.08) (width 0.25) (layer F.Cu) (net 3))
 (segment (start -5.08 -5.08) (end -5.08 -10.16) (width 0.25) (layer F.Cu) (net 3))
 (segment (start -5.51499 -0.38501) (end -5.54999 -0.35001) (width 0.25) (layer F.Cu) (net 4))
 (segment (start -1.125 1.95) (end -1.125 0.080514) (width 0.25) (layer F.Cu) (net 4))
 (segment (start -1.590524 -0.38501) (end -5.51499 -0.38501) (width 0.25) (layer F.Cu) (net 4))
 (segment (start -1.125 0.080514) (end -1.590524 -0.38501) (width 0.25) (layer F.Cu) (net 4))
 (segment (start -5.54999 -0.35001) (end -6.85001 -0.35001) (width 0.25) (layer F.Cu) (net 4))
 (segment (start -7.62 -1.12) (end -7.62 -2.54) (width 0.25) (layer F.Cu) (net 4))
 (segment (start -6.85001 -0.35001) (end -7.62 -1.12) (width 0.25) (layer F.Cu) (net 4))
 (segment (start -7.62 -2.54) (end -7.62 -5.08) (width 0.25) (layer F.Cu) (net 4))
 (segment (start -7.62 -5.08) (end -7.62 -10.16) (width 0.25) (layer F.Cu) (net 4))
 (segment (start 1.125 -1.415) (end 0 -2.54) (width 0.25) (layer B.Cu) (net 1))
 (segment (start 1.125 1.95) (end 1.125 -1.415) (width 0.25) (layer B.Cu) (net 1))
 (segment (start 0 -2.54) (end 0 -5.08) (width 0.25) (layer B.Cu) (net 1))
 (segment (start 0 -5.08) (end 0 -10.16) (width 0.25) (layer B.Cu) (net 1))
 (segment (start -2.54 -1.334486) (end -2.54 -2.54) (width 0.25) (layer B.Cu) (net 2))
 (segment (start -1.125 0.080514) (end -2.54 -1.334486) (width 0.25) (layer B.Cu) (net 2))
 (segment (start -1.125 1.95) (end -1.125 0.080514) (width 0.25) (layer B.Cu) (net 2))
 (segment (start -2.54 -2.54) (end -2.54 -5.08) (width 0.25) (layer B.Cu) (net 2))
 (segment (start -2.54 -5.08) (end -2.54 -10.16) (width 0.25) (layer B.Cu) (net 2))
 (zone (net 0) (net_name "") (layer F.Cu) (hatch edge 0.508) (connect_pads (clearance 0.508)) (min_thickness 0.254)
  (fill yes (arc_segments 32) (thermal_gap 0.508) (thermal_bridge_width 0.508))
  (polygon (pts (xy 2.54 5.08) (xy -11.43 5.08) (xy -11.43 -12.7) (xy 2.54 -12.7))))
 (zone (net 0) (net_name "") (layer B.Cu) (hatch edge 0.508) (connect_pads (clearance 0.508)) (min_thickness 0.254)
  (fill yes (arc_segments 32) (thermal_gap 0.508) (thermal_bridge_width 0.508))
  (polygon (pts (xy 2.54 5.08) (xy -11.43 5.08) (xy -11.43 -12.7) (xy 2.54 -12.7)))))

